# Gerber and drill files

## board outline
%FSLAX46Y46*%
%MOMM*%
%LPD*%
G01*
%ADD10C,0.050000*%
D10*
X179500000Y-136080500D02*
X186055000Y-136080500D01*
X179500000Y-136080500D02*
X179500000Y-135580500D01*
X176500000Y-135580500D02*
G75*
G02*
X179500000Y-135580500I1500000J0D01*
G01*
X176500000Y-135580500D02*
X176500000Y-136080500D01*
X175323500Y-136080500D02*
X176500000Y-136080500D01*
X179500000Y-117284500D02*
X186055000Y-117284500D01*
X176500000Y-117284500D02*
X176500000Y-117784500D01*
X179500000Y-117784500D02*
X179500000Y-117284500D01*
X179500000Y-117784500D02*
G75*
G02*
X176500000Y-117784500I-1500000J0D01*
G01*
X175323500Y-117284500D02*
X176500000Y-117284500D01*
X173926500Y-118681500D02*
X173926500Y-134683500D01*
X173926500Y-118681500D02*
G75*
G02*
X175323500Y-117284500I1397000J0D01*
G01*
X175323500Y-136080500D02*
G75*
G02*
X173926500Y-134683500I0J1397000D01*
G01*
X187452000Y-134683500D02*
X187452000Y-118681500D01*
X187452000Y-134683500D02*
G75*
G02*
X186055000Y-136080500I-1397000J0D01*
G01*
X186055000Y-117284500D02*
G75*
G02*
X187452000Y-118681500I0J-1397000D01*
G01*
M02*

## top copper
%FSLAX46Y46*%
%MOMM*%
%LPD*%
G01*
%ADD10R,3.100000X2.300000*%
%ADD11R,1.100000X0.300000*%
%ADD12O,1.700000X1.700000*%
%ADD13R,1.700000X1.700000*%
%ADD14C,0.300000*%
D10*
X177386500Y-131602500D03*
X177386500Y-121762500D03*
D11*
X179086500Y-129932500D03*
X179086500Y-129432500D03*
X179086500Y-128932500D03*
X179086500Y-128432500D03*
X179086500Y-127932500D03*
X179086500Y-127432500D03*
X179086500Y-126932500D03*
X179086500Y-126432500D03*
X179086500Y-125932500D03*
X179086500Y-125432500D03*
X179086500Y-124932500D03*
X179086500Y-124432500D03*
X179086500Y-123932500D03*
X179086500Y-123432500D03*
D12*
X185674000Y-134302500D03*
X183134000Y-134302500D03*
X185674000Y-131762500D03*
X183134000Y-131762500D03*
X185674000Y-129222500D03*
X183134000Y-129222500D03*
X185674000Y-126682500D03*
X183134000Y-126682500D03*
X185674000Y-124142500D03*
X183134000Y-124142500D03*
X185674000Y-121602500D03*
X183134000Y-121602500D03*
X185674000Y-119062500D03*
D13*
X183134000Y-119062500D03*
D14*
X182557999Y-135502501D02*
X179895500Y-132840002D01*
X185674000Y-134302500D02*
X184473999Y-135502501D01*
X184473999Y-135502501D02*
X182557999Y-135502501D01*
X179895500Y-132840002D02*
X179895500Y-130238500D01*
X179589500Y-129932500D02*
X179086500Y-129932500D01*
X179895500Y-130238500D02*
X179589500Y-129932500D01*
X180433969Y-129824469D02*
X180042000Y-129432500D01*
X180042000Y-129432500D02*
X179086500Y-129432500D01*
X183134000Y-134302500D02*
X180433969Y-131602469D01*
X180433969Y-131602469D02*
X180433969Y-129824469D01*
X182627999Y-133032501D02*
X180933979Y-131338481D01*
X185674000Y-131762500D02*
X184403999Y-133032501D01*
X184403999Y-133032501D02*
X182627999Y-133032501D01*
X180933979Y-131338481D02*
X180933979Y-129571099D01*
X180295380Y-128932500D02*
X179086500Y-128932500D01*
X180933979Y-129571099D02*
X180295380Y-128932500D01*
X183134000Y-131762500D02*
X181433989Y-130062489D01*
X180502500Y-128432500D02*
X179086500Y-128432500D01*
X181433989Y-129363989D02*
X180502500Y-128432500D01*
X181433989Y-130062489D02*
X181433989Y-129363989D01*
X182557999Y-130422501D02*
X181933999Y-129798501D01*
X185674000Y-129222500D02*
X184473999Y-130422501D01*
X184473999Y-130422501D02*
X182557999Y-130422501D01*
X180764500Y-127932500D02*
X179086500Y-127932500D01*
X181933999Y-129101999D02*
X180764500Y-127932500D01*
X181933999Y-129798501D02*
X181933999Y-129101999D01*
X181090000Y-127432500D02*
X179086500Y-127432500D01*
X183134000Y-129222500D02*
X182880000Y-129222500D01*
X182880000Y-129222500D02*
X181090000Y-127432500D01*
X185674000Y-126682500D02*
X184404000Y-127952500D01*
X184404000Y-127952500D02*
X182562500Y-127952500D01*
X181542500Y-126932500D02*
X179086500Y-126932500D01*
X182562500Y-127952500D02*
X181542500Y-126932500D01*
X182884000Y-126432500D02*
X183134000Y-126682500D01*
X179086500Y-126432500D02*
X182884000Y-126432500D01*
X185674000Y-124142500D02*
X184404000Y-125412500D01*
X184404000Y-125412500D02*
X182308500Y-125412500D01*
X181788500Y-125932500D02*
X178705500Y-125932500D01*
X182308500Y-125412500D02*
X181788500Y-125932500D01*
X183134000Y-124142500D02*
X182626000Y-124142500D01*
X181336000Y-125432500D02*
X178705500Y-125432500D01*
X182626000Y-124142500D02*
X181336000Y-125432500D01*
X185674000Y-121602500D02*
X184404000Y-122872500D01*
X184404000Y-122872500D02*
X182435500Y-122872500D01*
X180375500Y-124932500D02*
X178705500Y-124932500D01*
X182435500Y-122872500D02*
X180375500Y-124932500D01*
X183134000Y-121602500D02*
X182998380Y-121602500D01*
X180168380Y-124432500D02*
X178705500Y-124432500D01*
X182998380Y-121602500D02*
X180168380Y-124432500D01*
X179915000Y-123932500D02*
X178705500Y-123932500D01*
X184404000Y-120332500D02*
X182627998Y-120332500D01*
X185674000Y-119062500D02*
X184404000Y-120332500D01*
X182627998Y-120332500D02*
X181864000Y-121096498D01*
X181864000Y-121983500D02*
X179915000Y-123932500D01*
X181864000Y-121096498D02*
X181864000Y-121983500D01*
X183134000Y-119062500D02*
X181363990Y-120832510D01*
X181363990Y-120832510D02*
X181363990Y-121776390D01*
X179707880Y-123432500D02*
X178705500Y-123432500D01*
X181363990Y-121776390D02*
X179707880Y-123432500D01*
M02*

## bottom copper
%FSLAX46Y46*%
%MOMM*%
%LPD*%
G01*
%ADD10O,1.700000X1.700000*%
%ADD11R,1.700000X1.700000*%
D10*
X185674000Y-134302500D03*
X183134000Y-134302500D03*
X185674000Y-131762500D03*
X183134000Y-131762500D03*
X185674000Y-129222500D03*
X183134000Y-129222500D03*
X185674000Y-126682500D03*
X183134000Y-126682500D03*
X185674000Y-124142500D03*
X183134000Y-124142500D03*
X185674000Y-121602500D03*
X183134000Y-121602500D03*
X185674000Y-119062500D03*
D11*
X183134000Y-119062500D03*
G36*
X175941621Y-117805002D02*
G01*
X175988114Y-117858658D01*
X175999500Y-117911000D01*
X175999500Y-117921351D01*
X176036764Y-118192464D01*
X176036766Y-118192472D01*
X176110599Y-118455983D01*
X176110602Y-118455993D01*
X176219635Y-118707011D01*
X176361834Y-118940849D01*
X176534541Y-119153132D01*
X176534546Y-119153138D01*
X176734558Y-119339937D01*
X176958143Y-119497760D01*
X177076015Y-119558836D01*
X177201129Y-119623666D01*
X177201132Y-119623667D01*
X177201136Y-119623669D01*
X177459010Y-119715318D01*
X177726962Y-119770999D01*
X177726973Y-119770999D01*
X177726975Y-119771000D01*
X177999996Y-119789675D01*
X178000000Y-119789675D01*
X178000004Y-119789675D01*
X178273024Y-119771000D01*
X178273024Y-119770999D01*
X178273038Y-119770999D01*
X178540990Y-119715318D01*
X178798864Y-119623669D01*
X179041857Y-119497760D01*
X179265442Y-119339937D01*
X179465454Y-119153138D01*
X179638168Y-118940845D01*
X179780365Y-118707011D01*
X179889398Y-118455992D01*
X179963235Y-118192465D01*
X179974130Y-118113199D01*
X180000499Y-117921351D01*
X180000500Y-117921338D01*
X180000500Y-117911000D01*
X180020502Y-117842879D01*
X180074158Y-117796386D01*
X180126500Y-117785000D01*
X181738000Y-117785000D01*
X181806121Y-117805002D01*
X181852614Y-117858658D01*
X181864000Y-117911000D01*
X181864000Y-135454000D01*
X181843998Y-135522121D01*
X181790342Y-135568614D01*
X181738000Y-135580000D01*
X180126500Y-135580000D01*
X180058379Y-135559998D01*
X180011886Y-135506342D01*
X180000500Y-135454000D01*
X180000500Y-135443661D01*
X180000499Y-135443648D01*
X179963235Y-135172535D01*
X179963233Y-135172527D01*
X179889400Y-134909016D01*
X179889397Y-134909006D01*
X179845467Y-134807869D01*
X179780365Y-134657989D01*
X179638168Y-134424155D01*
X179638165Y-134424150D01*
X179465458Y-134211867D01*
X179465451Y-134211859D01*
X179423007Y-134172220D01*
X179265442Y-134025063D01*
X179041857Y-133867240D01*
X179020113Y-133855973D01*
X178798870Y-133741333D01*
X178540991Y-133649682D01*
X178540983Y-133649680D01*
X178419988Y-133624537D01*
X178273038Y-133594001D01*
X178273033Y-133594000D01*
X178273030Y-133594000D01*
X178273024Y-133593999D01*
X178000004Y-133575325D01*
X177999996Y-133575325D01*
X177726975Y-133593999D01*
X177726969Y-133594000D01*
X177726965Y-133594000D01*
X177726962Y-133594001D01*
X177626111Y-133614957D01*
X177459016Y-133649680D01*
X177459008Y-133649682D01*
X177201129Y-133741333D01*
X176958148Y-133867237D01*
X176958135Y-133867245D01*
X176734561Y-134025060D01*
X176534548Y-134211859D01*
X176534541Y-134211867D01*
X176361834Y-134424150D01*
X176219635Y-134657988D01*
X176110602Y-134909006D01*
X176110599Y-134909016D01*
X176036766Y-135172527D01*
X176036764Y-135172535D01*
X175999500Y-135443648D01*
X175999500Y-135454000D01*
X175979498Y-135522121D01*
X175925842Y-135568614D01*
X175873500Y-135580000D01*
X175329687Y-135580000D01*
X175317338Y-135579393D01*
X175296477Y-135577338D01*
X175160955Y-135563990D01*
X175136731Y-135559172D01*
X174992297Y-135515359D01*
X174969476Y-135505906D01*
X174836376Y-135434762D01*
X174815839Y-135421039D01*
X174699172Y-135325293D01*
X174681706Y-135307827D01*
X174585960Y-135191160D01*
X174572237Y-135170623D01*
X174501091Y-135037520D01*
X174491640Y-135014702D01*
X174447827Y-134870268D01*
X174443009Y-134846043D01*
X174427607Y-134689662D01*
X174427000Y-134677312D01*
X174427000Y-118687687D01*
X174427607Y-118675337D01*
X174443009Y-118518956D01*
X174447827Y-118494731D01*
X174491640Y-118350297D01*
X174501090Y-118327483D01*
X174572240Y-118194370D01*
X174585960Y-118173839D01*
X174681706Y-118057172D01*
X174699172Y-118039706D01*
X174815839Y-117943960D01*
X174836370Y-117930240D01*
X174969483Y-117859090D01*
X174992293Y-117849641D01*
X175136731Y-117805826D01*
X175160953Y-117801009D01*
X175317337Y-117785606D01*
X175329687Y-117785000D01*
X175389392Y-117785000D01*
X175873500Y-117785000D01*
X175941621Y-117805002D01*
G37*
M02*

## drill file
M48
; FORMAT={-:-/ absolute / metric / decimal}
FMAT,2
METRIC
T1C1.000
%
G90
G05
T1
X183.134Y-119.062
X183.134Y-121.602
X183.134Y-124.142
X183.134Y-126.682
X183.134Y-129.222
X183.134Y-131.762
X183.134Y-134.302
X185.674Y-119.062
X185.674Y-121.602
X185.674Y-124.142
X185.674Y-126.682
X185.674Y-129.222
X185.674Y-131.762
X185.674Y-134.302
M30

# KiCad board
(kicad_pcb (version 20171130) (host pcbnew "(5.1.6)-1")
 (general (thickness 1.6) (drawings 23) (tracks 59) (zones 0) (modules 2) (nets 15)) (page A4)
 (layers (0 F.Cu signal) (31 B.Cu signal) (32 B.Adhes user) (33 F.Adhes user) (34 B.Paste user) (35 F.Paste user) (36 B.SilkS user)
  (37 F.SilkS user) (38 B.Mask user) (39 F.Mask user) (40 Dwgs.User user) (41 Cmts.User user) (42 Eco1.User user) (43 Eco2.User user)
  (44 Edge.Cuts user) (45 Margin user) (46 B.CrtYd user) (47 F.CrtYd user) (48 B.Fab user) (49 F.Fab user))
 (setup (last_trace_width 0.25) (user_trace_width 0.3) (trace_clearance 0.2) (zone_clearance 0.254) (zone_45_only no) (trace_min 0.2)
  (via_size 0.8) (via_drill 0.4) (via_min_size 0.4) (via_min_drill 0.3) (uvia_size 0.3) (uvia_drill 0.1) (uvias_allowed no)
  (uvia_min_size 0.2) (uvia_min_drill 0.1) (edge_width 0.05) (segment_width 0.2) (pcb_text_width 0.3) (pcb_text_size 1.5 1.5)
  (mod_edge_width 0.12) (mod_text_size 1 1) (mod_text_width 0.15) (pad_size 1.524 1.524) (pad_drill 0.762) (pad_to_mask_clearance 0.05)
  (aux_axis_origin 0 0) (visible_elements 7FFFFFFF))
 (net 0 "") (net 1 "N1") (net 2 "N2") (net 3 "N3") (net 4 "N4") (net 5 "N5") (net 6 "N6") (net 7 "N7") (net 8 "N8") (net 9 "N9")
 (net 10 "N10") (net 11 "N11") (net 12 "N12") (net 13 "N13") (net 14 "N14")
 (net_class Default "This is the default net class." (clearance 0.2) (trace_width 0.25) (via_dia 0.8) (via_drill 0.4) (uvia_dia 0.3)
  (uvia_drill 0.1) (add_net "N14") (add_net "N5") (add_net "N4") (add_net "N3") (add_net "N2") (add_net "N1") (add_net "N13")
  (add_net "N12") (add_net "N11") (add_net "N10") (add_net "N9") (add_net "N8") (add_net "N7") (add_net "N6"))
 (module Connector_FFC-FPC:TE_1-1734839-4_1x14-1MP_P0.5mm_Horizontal (layer F.Cu) (at 177.7365 126.6825 270)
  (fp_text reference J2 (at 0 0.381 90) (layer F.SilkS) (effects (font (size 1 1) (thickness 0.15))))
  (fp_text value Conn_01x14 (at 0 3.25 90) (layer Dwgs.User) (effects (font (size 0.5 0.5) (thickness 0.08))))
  (pad MP smd rect (at 4.92 0.35 270) (size 2.3 3.1) (layers F.Cu F.Paste F.Mask))
  (pad MP smd rect (at -4.92 0.35 270) (size 2.3 3.1) (layers F.Cu F.Paste F.Mask))
  (pad 14 smd rect (at 3.25 -1.35 270) (size 0.3 1.1) (layers F.Cu F.Paste F.Mask) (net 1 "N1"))
  (pad 13 smd rect (at 2.75 -1.35 270) (size 0.3 1.1) (layers F.Cu F.Paste F.Mask) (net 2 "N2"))
  (pad 12 smd rect (at 2.25 -1.35 270) (size 0.3 1.1) (layers F.Cu F.Paste F.Mask) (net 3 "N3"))
  (pad 11 smd rect (at 1.75 -1.35 270) (size 0.3 1.1) (layers F.Cu F.Paste F.Mask) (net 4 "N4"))
  (pad 10 smd rect (at 1.25 -1.35 270) (size 0.3 1.1) (layers F.Cu F.Paste F.Mask) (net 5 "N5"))
  (pad 9 smd rect (at 0.75 -1.35 270) (size 0.3 1.1) (layers F.Cu F.Paste F.Mask) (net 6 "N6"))
  (pad 8 smd rect (at 0.25 -1.35 270) (size 0.3 1.1) (layers F.Cu F.Paste F.Mask) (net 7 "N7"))
  (pad 7 smd rect (at -0.25 -1.35 270) (size 0.3 1.1) (layers F.Cu F.Paste F.Mask) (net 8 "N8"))
  (pad 6 smd rect (at -0.75 -1.35 270) (size 0.3 1.1) (layers F.Cu F.Paste F.Mask) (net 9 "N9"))
  (pad 5 smd rect (at -1.25 -1.35 270) (size 0.3 1.1) (layers F.Cu F.Paste F.Mask) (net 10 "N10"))
  (pad 4 smd rect (at -1.75 -1.35 270) (size 0.3 1.1) (layers F.Cu F.Paste F.Mask) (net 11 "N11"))
  (pad 3 smd rect (at -2.25 -1.35 270) (size 0.3 1.1) (layers F.Cu F.Paste F.Mask) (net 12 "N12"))
  (pad 2 smd rect (at -2.75 -1.35 270) (size 0.3 1.1) (layers F.Cu F.Paste F.Mask) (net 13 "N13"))
  (pad 1 smd rect (at -3.25 -1.35 270) (size 0.3 1.1) (layers F.Cu F.Paste F.Mask) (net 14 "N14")))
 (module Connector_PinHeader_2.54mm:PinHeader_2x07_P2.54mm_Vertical (layer F.Cu) (at 183.134 119.0625)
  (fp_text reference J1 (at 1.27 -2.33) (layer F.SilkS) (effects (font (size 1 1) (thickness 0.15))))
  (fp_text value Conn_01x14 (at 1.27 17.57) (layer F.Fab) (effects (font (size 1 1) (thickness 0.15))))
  (pad 14 thru_hole oval (at 2.54 15.24) (size 1.7 1.7) (drill 1) (layers *.Cu *.Mask) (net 1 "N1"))
  (pad 13 thru_hole oval (at 0 15.24) (size 1.7 1.7) (drill 1) (layers *.Cu *.Mask) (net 2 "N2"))
  (pad 12 thru_hole oval (at 2.54 12.7) (size 1.7 1.7) (drill 1) (layers *.Cu *.Mask) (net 3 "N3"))
  (pad 11 thru_hole oval (at 0 12.7) (size 1.7 1.7) (drill 1) (layers *.Cu *.Mask) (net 4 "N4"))
  (pad 10 thru_hole oval (at 2.54 10.16) (size 1.7 1.7) (drill 1) (layers *.Cu *.Mask) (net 5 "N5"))
  (pad 9 thru_hole oval (at 0 10.16) (size 1.7 1.7) (drill 1) (layers *.Cu *.Mask) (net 6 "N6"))
  (pad 8 thru_hole oval (at 2.54 7.62) (size 1.7 1.7) (drill 1) (layers *.Cu *.Mask) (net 7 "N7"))
  (pad 7 thru_hole oval (at 0 7.62) (size 1.7 1.7) (drill 1) (layers *.Cu *.Mask) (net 8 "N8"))
  (pad 6 thru_hole oval (at 2.54 5.08) (size 1.7 1.7) (drill 1) (layers *.Cu *.Mask) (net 9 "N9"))
  (pad 5 thru_hole oval (at 0 5.08) (size 1.7 1.7) (drill 1) (layers *.Cu *.Mask) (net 10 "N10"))
  (pad 4 thru_hole oval (at 2.54 2.54) (size 1.7 1.7) (drill 1) (layers *.Cu *.Mask) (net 11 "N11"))
  (pad 3 thru_hole oval (at 0 2.54) (size 1.7 1.7) (drill 1) (layers *.Cu *.Mask) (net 12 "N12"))
  (pad 2 thru_hole oval (at 2.54 0) (size 1.7 1.7) (drill 1) (layers *.Cu *.Mask) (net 13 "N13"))
  (pad 1 thru_hole rect (at 0 0) (size 1.7 1.7) (drill 1) (layers *.Cu *.Mask) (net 14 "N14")))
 (gr_line (start 179.5 136.0805) (end 186.055 136.0805) (layer Edge.Cuts) (width 0.05))
 (gr_line (start 179.5 136.0805) (end 179.5 135.5805) (layer Edge.Cuts) (width 0.05))
 (gr_arc (start 178 135.5805) (end 179.5 135.5805) (angle -180) (layer Edge.Cuts) (width 0.05))
 (gr_line (start 176.5 135.5805) (end 176.5 136.0805) (layer Edge.Cuts) (width 0.05))
 (gr_line (start 175.3235 136.0805) (end 176.5 136.0805) (layer Edge.Cuts) (width 0.05))
 (gr_line (start 179.5 117.2845) (end 186.055 117.2845) (layer Edge.Cuts) (width 0.05))
 (gr_line (start 176.5 117.2845) (end 176.5 117.7845) (layer Edge.Cuts) (width 0.05))
 (gr_line (start 179.5 117.7845) (end 179.5 117.2845) (layer Edge.Cuts) (width 0.05))
 (gr_arc (start 178 117.7845) (end 176.5 117.7845) (angle -180) (layer Edge.Cuts) (width 0.05))
 (gr_line (start 175.3235 117.2845) (end 176.5 117.2845) (layer Edge.Cuts) (width 0.05))
 (gr_line (start 173.9265 118.6815) (end 173.9265 134.6835) (layer Edge.Cuts) (width 0.05))
 (gr_arc (start 175.3235 118.6815) (end 175.3235 117.2845) (angle -90) (layer Edge.Cuts) (width 0.05))
 (gr_arc (start 175.3235 134.6835) (end 173.9265 134.6835) (angle -90) (layer Edge.Cuts) (width 0.05))
 (gr_line (start 187.452 134.6835) (end 187.452 118.6815) (layer Edge.Cuts) (width 0.05))
 (gr_arc (start 186.055 134.6835) (end 186.055 136.0805) (angle -90) (layer Edge.Cuts) (width 0.05))
 (gr_arc (start 186.055 118.6815) (end 187.452 118.6815) (angle -90) (layer Edge.Cuts) (width 0.05))
 (segment (start 182.557999 135.502501) (end 179.8955 132.840002) (width 0.3) (layer F.Cu) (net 1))
 (segment (start 185.674 134.3025) (end 184.473999 135.502501) (width 0.3) (layer F.Cu) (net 1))
 (segment (start 184.473999 135.502501) (end 182.557999 135.502501) (width 0.3) (layer F.Cu) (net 1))
 (segment (start 179.8955 132.840002) (end 179.8955 130.2385) (width 0.3) (layer F.Cu) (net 1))
 (segment (start 179.5895 129.9325) (end 179.0865 129.9325) (width 0.3) (layer F.Cu) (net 1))
 (segment (start 179.8955 130.2385) (end 179.5895 129.9325) (width 0.3) (layer F.Cu) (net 1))
 (segment (start 180.433969 129.824469) (end 180.042 129.4325) (width 0.3) (layer F.Cu) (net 2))
 (segment (start 180.042 129.4325) (end 179.0865 129.4325) (width 0.3) (layer F.Cu) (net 2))
 (segment (start 183.134 134.3025) (end 180.433969 131.602469) (width 0.3) (layer F.Cu) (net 2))
 (segment (start 180.433969 131.602469) (end 180.433969 129.824469) (width 0.3) (layer F.Cu) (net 2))
 (segment (start 182.627999 133.032501) (end 180.933979 131.338481) (width 0.3) (layer F.Cu) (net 3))
 (segment (start 185.674 131.7625) (end 184.403999 133.032501) (width 0.3) (layer F.Cu) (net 3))
 (segment (start 184.403999 133.032501) (end 182.627999 133.032501) (width 0.3) (layer F.Cu) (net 3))
 (segment (start 180.933979 131.338481) (end 180.933979 129.571099) (width 0.3) (layer F.Cu) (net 3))
 (segment (start 180.29538 128.9325) (end 179.0865 128.9325) (width 0.3) (layer F.Cu) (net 3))
 (segment (start 180.933979 129.571099) (end 180.29538 128.9325) (width 0.3) (layer F.Cu) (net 3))
 (segment (start 183.134 131.7625) (end 181.433989 130.062489) (width 0.3) (layer F.Cu) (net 4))
 (segment (start 180.5025 128.4325) (end 179.0865 128.4325) (width 0.3) (layer F.Cu) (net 4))
 (segment (start 181.433989 129.363989) (end 180.5025 128.4325) (width 0.3) (layer F.Cu) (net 4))
 (segment (start 181.433989 130.062489) (end 181.433989 129.363989) (width 0.3) (layer F.Cu) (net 4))
 (segment (start 182.557999 130.422501) (end 181.933999 129.798501) (width 0.3) (layer F.Cu) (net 5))
 (segment (start 185.674 129.2225) (end 184.473999 130.422501) (width 0.3) (layer F.Cu) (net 5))
 (segment (start 184.473999 130.422501) (end 182.557999 130.422501) (width 0.3) (layer F.Cu) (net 5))
 (segment (start 180.7645 127.9325) (end 179.0865 127.9325) (width 0.3) (layer F.Cu) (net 5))
 (segment (start 181.933999 129.101999) (end 180.7645 127.9325) (width 0.3) (layer F.Cu) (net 5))
 (segment (start 181.933999 129.798501) (end 181.933999 129.101999) (width 0.3) (layer F.Cu) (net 5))
 (segment (start 181.09 127.4325) (end 179.0865 127.4325) (width 0.3) (layer F.Cu) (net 6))
 (segment (start 183.134 129.2225) (end 182.88 129.2225) (width 0.3) (layer F.Cu) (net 6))
 (segment (start 182.88 129.2225) (end 181.09 127.4325) (width 0.3) (layer F.Cu) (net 6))
 (segment (start 185.674 126.6825) (end 184.404 127.9525) (width 0.3) (layer F.Cu) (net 7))
 (segment (start 184.404 127.9525) (end 182.5625 127.9525) (width 0.3) (layer F.Cu) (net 7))
 (segment (start 181.5425 126.9325) (end 179.0865 126.9325) (width 0.3) (layer F.Cu) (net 7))
 (segment (start 182.5625 127.9525) (end 181.5425 126.9325) (width 0.3) (layer F.Cu) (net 7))
 (segment (start 182.884 126.4325) (end 183.134 126.6825) (width 0.3) (layer F.Cu) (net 8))
 (segment (start 179.0865 126.4325) (end 182.884 126.4325) (width 0.3) (layer F.Cu) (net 8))
 (segment (start 185.674 124.1425) (end 184.404 125.4125) (width 0.3) (layer F.Cu) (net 9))
 (segment (start 184.404 125.4125) (end 182.3085 125.4125) (width 0.3) (layer F.Cu) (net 9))
 (segment (start 181.7885 125.9325) (end 178.7055 125.9325) (width 0.3) (layer F.Cu) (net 9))
 (segment (start 182.3085 125.4125) (end 181.7885 125.9325) (width 0.3) (layer F.Cu) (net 9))
 (segment (start 183.134 124.1425) (end 182.626 124.1425) (width 0.3) (layer F.Cu) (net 10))
 (segment (start 181.336 125.4325) (end 178.7055 125.4325) (width 0.3) (layer F.Cu) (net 10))
 (segment (start 182.626 124.1425) (end 181.336 125.4325) (width 0.3) (layer F.Cu) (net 10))
 (segment (start 185.674 121.6025) (end 184.404 122.8725) (width 0.3) (layer F.Cu) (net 11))
 (segment (start 184.404 122.8725) (end 182.4355 122.8725) (width 0.3) (layer F.Cu) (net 11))
 (segment (start 180.3755 124.9325) (end 178.7055 124.9325) (width 0.3) (layer F.Cu) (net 11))
 (segment (start 182.4355 122.8725) (end 180.3755 124.9325) (width 0.3) (layer F.Cu) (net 11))
 (segment (start 183.134 121.6025) (end 182.99838 121.6025) (width 0.3) (layer F.Cu) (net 12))
 (segment (start 180.16838 124.4325) (end 178.7055 124.4325) (width 0.3) (layer F.Cu) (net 12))
 (segment (start 182.99838 121.6025) (end 180.16838 124.4325) (width 0.3) (layer F.Cu) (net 12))
 (segment (start 179.915 123.9325) (end 178.7055 123.9325) (width 0.3) (layer F.Cu) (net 13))
 (segment (start 184.404 120.3325) (end 182.627998 120.3325) (width 0.3) (layer F.Cu) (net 13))
 (segment (start 185.674 119.0625) (end 184.404 120.3325) (width 0.3) (layer F.Cu) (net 13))
 (segment (start 182.627998 120.3325) (end 181.864 121.096498) (width 0.3) (layer F.Cu) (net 13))
 (segment (start 181.864 121.9835) (end 179.915 123.9325) (width 0.3) (layer F.Cu) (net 13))
 (segment (start 181.864 121.096498) (end 181.864 121.9835) (width 0.3) (layer F.Cu) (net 13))
 (segment (start 183.134 119.0625) (end 181.36399 120.83251) (width 0.3) (layer F.Cu) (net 14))
 (segment (start 181.36399 120.83251) (end 181.36399 121.77639) (width 0.3) (layer F.Cu) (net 14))
 (segment (start 179.70788 123.4325) (end 178.7055 123.4325) (width 0.3) (layer F.Cu) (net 14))
 (segment (start 181.36399 121.77639) (end 179.70788 123.4325) (width 0.3) (layer F.Cu) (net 14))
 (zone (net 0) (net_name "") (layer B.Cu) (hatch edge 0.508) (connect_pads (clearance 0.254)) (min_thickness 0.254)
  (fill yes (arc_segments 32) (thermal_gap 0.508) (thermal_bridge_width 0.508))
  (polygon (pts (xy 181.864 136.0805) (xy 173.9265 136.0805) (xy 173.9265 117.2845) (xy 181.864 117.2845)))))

